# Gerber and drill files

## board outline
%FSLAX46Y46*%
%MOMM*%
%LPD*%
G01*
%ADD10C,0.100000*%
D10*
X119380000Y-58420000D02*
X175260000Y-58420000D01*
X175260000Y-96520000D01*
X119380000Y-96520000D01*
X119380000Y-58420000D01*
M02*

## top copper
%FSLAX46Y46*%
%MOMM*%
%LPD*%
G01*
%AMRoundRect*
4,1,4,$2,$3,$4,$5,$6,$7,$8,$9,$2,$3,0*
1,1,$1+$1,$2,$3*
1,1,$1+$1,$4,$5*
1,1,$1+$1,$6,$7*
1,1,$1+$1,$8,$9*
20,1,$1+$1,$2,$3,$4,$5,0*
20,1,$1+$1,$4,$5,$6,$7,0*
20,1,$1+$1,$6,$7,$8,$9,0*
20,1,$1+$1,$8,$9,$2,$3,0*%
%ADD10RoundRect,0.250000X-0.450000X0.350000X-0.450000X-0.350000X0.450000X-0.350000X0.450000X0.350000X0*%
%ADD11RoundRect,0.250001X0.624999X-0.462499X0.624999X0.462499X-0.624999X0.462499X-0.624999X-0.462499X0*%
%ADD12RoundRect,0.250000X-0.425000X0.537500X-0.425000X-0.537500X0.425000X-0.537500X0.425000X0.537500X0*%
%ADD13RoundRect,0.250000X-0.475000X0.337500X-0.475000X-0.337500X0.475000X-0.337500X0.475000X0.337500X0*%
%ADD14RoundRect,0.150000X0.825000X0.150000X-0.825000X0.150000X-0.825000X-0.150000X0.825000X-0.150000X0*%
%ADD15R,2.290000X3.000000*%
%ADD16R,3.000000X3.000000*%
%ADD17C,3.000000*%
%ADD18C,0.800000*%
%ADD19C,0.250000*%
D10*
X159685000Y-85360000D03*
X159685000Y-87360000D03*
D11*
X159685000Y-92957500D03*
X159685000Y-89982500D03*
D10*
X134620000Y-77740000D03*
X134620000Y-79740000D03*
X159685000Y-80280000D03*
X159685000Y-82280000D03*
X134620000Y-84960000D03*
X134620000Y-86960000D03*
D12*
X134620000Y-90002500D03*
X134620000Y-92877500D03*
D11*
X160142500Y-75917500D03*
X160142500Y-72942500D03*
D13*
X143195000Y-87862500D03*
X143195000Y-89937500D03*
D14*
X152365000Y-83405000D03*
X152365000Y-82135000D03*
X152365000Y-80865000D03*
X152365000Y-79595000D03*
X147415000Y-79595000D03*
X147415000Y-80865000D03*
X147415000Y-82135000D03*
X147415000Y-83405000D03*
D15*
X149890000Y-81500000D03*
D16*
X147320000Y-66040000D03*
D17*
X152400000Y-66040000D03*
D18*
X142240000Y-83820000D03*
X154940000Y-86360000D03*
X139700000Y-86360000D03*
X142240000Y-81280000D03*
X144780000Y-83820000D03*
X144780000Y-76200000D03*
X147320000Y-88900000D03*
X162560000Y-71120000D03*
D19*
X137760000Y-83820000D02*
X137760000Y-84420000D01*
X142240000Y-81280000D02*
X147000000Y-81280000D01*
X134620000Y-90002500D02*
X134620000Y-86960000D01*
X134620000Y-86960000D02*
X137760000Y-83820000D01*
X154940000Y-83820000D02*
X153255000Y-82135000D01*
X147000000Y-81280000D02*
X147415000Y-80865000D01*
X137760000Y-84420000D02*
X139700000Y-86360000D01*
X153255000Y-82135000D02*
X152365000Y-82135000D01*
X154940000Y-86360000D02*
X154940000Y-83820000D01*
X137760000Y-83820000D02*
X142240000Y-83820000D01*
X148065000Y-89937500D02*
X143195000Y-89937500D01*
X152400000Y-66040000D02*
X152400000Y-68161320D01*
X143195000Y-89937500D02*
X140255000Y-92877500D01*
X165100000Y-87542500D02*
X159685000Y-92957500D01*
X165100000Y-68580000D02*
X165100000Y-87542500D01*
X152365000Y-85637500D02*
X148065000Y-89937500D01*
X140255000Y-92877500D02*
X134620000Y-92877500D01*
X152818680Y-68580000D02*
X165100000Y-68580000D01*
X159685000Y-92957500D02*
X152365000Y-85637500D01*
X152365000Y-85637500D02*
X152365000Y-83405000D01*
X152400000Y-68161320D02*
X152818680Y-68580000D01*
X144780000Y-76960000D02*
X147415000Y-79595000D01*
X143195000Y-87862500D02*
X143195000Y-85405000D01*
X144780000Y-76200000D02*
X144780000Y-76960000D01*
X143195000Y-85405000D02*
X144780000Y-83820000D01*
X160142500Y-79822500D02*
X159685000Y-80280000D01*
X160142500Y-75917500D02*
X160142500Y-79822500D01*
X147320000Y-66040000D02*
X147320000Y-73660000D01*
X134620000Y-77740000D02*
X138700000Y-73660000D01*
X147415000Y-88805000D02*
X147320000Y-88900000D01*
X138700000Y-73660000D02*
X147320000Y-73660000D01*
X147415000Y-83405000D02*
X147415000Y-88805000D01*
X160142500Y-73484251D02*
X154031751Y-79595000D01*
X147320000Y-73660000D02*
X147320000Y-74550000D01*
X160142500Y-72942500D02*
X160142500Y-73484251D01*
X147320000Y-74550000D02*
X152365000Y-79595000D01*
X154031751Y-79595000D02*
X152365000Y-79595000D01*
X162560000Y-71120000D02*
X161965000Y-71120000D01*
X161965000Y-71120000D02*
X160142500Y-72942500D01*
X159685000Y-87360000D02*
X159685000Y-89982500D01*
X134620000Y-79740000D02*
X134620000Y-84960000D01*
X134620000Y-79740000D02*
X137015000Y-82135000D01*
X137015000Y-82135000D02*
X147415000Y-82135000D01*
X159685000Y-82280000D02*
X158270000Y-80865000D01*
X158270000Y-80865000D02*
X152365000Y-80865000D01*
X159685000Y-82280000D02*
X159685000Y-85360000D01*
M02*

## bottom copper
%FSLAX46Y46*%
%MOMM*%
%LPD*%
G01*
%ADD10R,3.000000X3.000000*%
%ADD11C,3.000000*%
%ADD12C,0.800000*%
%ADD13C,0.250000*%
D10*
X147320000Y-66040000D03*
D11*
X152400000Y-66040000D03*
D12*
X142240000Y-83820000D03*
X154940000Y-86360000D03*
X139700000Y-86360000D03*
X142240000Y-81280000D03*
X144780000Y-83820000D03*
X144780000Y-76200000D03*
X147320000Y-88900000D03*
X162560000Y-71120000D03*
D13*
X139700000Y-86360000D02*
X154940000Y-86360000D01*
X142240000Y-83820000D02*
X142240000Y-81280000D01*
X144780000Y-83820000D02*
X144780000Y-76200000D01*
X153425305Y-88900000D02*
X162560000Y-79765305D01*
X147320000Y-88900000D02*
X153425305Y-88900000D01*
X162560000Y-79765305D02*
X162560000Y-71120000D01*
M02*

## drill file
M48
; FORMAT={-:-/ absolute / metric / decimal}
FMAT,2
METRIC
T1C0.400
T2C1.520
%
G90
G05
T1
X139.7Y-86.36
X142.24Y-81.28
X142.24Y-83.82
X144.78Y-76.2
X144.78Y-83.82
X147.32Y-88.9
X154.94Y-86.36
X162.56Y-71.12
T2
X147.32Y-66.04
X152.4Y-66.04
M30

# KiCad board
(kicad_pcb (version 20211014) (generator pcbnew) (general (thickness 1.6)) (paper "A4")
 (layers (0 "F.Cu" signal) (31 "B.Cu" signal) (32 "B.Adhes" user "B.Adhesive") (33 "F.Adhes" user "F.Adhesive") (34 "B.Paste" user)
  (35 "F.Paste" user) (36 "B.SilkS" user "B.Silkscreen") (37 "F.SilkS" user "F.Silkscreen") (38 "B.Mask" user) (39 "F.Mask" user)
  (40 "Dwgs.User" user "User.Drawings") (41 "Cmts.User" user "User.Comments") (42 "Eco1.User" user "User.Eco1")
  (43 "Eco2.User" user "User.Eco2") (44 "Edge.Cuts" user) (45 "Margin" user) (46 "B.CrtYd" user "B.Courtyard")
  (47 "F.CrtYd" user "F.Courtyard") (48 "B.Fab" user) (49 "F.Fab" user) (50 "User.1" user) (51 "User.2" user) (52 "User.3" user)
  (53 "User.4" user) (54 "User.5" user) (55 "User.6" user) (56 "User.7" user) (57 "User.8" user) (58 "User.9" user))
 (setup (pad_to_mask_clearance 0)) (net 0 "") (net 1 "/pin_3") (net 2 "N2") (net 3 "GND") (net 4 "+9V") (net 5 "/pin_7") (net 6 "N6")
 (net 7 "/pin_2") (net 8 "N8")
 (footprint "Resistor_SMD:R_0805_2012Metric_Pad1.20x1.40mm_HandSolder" (layer "F.Cu") (at 159.685 86.36 -90)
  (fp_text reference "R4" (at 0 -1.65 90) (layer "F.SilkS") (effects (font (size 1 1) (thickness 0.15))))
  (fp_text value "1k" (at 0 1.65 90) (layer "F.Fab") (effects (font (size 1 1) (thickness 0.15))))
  (pad "1" smd roundrect (at -1 0 270) (size 1.2 1.4) (layers "F.Cu" "F.Paste" "F.Mask") (roundrect_rratio 0.208333) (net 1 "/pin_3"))
  (pad "2" smd roundrect (at 1 0 270) (size 1.2 1.4) (layers "F.Cu" "F.Paste" "F.Mask") (roundrect_rratio 0.208333) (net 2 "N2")))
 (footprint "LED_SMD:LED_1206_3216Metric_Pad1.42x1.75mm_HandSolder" (layer "F.Cu") (at 159.685 91.47 90)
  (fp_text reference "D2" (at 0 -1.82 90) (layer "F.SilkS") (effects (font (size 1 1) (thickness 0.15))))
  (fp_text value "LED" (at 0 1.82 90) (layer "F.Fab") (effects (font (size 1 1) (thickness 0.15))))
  (pad "1" smd roundrect (at -1.4875 0 90) (size 1.425 1.75) (layers "F.Cu" "F.Paste" "F.Mask") (roundrect_rratio 0.175439) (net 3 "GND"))
  (pad "2" smd roundrect (at 1.4875 0 90) (size 1.425 1.75) (layers "F.Cu" "F.Paste" "F.Mask") (roundrect_rratio 0.175439) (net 2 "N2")))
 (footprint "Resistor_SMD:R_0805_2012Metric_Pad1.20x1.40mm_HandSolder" (layer "F.Cu") (at 134.62 78.74 -90)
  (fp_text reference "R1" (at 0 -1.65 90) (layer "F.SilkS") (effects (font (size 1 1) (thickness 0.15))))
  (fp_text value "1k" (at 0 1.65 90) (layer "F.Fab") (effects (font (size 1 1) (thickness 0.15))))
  (pad "1" smd roundrect (at -1 0 270) (size 1.2 1.4) (layers "F.Cu" "F.Paste" "F.Mask") (roundrect_rratio 0.208333) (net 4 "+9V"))
  (pad "2" smd roundrect (at 1 0 270) (size 1.2 1.4) (layers "F.Cu" "F.Paste" "F.Mask") (roundrect_rratio 0.208333) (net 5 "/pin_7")))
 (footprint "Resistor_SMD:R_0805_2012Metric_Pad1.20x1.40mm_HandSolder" (layer "F.Cu") (at 159.685 81.28 -90)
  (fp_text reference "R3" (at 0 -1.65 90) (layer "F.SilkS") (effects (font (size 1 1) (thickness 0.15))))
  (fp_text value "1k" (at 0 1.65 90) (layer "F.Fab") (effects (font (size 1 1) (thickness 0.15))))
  (pad "1" smd roundrect (at -1 0 270) (size 1.2 1.4) (layers "F.Cu" "F.Paste" "F.Mask") (roundrect_rratio 0.208333) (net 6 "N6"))
  (pad "2" smd roundrect (at 1 0 270) (size 1.2 1.4) (layers "F.Cu" "F.Paste" "F.Mask") (roundrect_rratio 0.208333) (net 1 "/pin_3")))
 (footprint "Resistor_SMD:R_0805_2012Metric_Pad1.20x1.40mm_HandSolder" (layer "F.Cu") (at 134.62 85.96 -90)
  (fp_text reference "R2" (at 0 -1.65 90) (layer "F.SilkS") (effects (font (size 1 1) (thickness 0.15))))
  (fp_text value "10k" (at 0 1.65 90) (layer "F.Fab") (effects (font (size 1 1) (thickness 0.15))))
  (pad "1" smd roundrect (at -1 0 270) (size 1.2 1.4) (layers "F.Cu" "F.Paste" "F.Mask") (roundrect_rratio 0.208333) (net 5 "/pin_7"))
  (pad "2" smd roundrect (at 1 0 270) (size 1.2 1.4) (layers "F.Cu" "F.Paste" "F.Mask") (roundrect_rratio 0.208333) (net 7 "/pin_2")))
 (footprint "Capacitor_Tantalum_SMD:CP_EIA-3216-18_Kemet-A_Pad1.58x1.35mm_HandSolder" (layer "F.Cu") (at 134.62 91.44 -90)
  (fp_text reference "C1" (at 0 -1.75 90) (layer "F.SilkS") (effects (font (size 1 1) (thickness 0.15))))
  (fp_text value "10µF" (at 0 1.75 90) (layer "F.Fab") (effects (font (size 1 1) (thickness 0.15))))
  (pad "1" smd roundrect (at -1.4375 0 270) (size 1.575 1.35) (layers "F.Cu" "F.Paste" "F.Mask") (roundrect_rratio 0.185185)
   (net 7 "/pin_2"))
  (pad "2" smd roundrect (at 1.4375 0 270) (size 1.575 1.35) (layers "F.Cu" "F.Paste" "F.Mask") (roundrect_rratio 0.185185) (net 3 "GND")))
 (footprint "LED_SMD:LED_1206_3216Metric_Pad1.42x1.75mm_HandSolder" (layer "F.Cu") (at 160.1425 74.43 90)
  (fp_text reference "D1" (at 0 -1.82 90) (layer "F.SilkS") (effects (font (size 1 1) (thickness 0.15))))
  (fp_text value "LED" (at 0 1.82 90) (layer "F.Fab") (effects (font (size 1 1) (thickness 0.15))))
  (pad "1" smd roundrect (at -1.4875 0 90) (size 1.425 1.75) (layers "F.Cu" "F.Paste" "F.Mask") (roundrect_rratio 0.175439) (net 6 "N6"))
  (pad "2" smd roundrect (at 1.4875 0 90) (size 1.425 1.75) (layers "F.Cu" "F.Paste" "F.Mask") (roundrect_rratio 0.175439) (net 4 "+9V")))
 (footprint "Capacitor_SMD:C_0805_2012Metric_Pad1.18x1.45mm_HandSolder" (layer "F.Cu") (at 143.195 88.9 -90)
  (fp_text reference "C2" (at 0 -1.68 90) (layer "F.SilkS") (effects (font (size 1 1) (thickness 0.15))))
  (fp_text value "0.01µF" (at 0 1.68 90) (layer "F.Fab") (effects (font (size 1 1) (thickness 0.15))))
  (pad "1" smd roundrect (at -1.0375 0 270) (size 1.175 1.45) (layers "F.Cu" "F.Paste" "F.Mask") (roundrect_rratio 0.212766) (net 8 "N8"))
  (pad "2" smd roundrect (at 1.0375 0 270) (size 1.175 1.45) (layers "F.Cu" "F.Paste" "F.Mask") (roundrect_rratio 0.212766) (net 3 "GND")))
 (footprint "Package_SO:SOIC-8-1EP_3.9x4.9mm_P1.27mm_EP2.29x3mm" (layer "F.Cu") (at 149.89 81.5 180)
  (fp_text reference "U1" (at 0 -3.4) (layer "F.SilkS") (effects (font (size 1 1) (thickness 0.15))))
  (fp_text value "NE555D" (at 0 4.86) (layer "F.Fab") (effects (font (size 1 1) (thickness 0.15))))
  (pad "" smd roundrect (at 0.57 0.75 180) (size 0.92 1.21) (layers "F.Paste") (roundrect_rratio 0.25))
  (pad "" smd roundrect (at 0.57 -0.75 180) (size 0.92 1.21) (layers "F.Paste") (roundrect_rratio 0.25))
  (pad "" smd roundrect (at -0.57 0.75 180) (size 0.92 1.21) (layers "F.Paste") (roundrect_rratio 0.25))
  (pad "" smd roundrect (at -0.57 -0.75 180) (size 0.92 1.21) (layers "F.Paste") (roundrect_rratio 0.25))
  (pad "1" smd roundrect (at -2.475 -1.905 180) (size 1.95 0.6) (layers "F.Cu" "F.Paste" "F.Mask") (roundrect_rratio 0.25) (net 3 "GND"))
  (pad "2" smd roundrect (at -2.475 -0.635 180) (size 1.95 0.6) (layers "F.Cu" "F.Paste" "F.Mask") (roundrect_rratio 0.25) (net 7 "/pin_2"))
  (pad "3" smd roundrect (at -2.475 0.635 180) (size 1.95 0.6) (layers "F.Cu" "F.Paste" "F.Mask") (roundrect_rratio 0.25) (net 1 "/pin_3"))
  (pad "4" smd roundrect (at -2.475 1.905 180) (size 1.95 0.6) (layers "F.Cu" "F.Paste" "F.Mask") (roundrect_rratio 0.25) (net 4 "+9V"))
  (pad "5" smd roundrect (at 2.475 1.905 180) (size 1.95 0.6) (layers "F.Cu" "F.Paste" "F.Mask") (roundrect_rratio 0.25) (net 8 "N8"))
  (pad "6" smd roundrect (at 2.475 0.635 180) (size 1.95 0.6) (layers "F.Cu" "F.Paste" "F.Mask") (roundrect_rratio 0.25) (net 7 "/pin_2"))
  (pad "7" smd roundrect (at 2.475 -0.635 180) (size 1.95 0.6) (layers "F.Cu" "F.Paste" "F.Mask") (roundrect_rratio 0.25) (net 5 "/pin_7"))
  (pad "8" smd roundrect (at 2.475 -1.905 180) (size 1.95 0.6) (layers "F.Cu" "F.Paste" "F.Mask") (roundrect_rratio 0.25) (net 4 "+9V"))
  (pad "9" smd rect (at 0 0 180) (size 2.29 3) (layers "F.Cu" "F.Mask")))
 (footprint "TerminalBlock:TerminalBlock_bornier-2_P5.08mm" (layer "F.Cu") (at 147.32 66.04)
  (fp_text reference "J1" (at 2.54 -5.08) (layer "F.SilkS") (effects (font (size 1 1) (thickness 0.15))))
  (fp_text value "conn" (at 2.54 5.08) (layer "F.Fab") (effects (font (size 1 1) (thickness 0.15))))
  (pad "1" thru_hole rect (at 0 0) (size 3 3) (drill 1.52) (layers *.Cu *.Mask) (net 4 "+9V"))
  (pad "2" thru_hole circle (at 5.08 0) (size 3 3) (drill 1.52) (layers *.Cu *.Mask) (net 3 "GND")))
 (gr_rect (start 119.38 58.42) (end 175.26 96.52) (layer "Edge.Cuts") (width 0.1) (fill none))
 (segment (start 137.76 83.82) (end 137.76 84.42) (width 0.25) (layer "F.Cu") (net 7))
 (segment (start 142.24 81.28) (end 147 81.28) (width 0.25) (layer "F.Cu") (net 7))
 (segment (start 134.62 90.0025) (end 134.62 86.96) (width 0.25) (layer "F.Cu") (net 7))
 (segment (start 134.62 86.96) (end 137.76 83.82) (width 0.25) (layer "F.Cu") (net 7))
 (segment (start 154.94 83.82) (end 153.255 82.135) (width 0.25) (layer "F.Cu") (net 7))
 (segment (start 147 81.28) (end 147.415 80.865) (width 0.25) (layer "F.Cu") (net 7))
 (segment (start 137.76 84.42) (end 139.7 86.36) (width 0.25) (layer "F.Cu") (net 7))
 (segment (start 153.255 82.135) (end 152.365 82.135) (width 0.25) (layer "F.Cu") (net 7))
 (segment (start 154.94 86.36) (end 154.94 83.82) (width 0.25) (layer "F.Cu") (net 7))
 (segment (start 137.76 83.82) (end 142.24 83.82) (width 0.25) (layer "F.Cu") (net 7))
 (via (at 142.24 83.82) (size 0.8) (drill 0.4) (layers "F.Cu" "B.Cu") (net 7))
 (via (at 154.94 86.36) (size 0.8) (drill 0.4) (layers "F.Cu" "B.Cu") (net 7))
 (via (at 139.7 86.36) (size 0.8) (drill 0.4) (layers "F.Cu" "B.Cu") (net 7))
 (via (at 142.24 81.28) (size 0.8) (drill 0.4) (layers "F.Cu" "B.Cu") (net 7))
 (segment (start 139.7 86.36) (end 154.94 86.36) (width 0.25) (layer "B.Cu") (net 7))
 (segment (start 142.24 83.82) (end 142.24 81.28) (width 0.25) (layer "B.Cu") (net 7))
 (segment (start 148.065 89.9375) (end 143.195 89.9375) (width 0.25) (layer "F.Cu") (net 3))
 (segment (start 152.4 66.04) (end 152.4 68.16132) (width 0.25) (layer "F.Cu") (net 3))
 (segment (start 143.195 89.9375) (end 140.255 92.8775) (width 0.25) (layer "F.Cu") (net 3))
 (segment (start 165.1 87.5425) (end 159.685 92.9575) (width 0.25) (layer "F.Cu") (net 3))
 (segment (start 165.1 68.58) (end 165.1 87.5425) (width 0.25) (layer "F.Cu") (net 3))
 (segment (start 152.365 85.6375) (end 148.065 89.9375) (width 0.25) (layer "F.Cu") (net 3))
 (segment (start 140.255 92.8775) (end 134.62 92.8775) (width 0.25) (layer "F.Cu") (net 3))
 (segment (start 152.81868 68.58) (end 165.1 68.58) (width 0.25) (layer "F.Cu") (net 3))
 (segment (start 159.685 92.9575) (end 152.365 85.6375) (width 0.25) (layer "F.Cu") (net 3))
 (segment (start 152.365 85.6375) (end 152.365 83.405) (width 0.25) (layer "F.Cu") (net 3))
 (segment (start 152.4 68.16132) (end 152.81868 68.58) (width 0.25) (layer "F.Cu") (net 3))
 (segment (start 144.78 76.96) (end 147.415 79.595) (width 0.25) (layer "F.Cu") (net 8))
 (segment (start 143.195 87.8625) (end 143.195 85.405) (width 0.25) (layer "F.Cu") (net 8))
 (segment (start 144.78 76.2) (end 144.78 76.96) (width 0.25) (layer "F.Cu") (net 8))
 (segment (start 143.195 85.405) (end 144.78 83.82) (width 0.25) (layer "F.Cu") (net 8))
 (via (at 144.78 83.82) (size 0.8) (drill 0.4) (layers "F.Cu" "B.Cu") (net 8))
 (via (at 144.78 76.2) (size 0.8) (drill 0.4) (layers "F.Cu" "B.Cu") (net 8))
 (segment (start 144.78 83.82) (end 144.78 76.2) (width 0.25) (layer "B.Cu") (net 8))
 (segment (start 160.1425 79.8225) (end 159.685 80.28) (width 0.25) (layer "F.Cu") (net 6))
 (segment (start 160.1425 75.9175) (end 160.1425 79.8225) (width 0.25) (layer "F.Cu") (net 6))
 (segment (start 147.32 66.04) (end 147.32 73.66) (width 0.25) (layer "F.Cu") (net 4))
 (segment (start 134.62 77.74) (end 138.7 73.66) (width 0.25) (layer "F.Cu") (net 4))
 (segment (start 147.415 88.805) (end 147.32 88.9) (width 0.25) (layer "F.Cu") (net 4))
 (segment (start 138.7 73.66) (end 147.32 73.66) (width 0.25) (layer "F.Cu") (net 4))
 (segment (start 147.415 83.405) (end 147.415 88.805) (width 0.25) (layer "F.Cu") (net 4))
 (segment (start 160.1425 73.484251) (end 154.031751 79.595) (width 0.25) (layer "F.Cu") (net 4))
 (segment (start 147.32 73.66) (end 147.32 74.55) (width 0.25) (layer "F.Cu") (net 4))
 (segment (start 160.1425 72.9425) (end 160.1425 73.484251) (width 0.25) (layer "F.Cu") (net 4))
 (segment (start 147.32 74.55) (end 152.365 79.595) (width 0.25) (layer "F.Cu") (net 4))
 (segment (start 154.031751 79.595) (end 152.365 79.595) (width 0.25) (layer "F.Cu") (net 4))
 (segment (start 162.56 71.12) (end 161.965 71.12) (width 0.25) (layer "F.Cu") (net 4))
 (segment (start 161.965 71.12) (end 160.1425 72.9425) (width 0.25) (layer "F.Cu") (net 4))
 (via (at 147.32 88.9) (size 0.8) (drill 0.4) (layers "F.Cu" "B.Cu") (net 4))
 (via (at 162.56 71.12) (size 0.8) (drill 0.4) (layers "F.Cu" "B.Cu") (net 4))
 (segment (start 153.425305 88.9) (end 162.56 79.765305) (width 0.25) (layer "B.Cu") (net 4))
 (segment (start 147.32 88.9) (end 153.425305 88.9) (width 0.25) (layer "B.Cu") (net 4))
 (segment (start 162.56 79.765305) (end 162.56 71.12) (width 0.25) (layer "B.Cu") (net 4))
 (segment (start 159.685 87.36) (end 159.685 89.9825) (width 0.25) (layer "F.Cu") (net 2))
 (segment (start 134.62 79.74) (end 134.62 84.96) (width 0.25) (layer "F.Cu") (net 5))
 (segment (start 134.62 79.74) (end 137.015 82.135) (width 0.25) (layer "F.Cu") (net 5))
 (segment (start 137.015 82.135) (end 147.415 82.135) (width 0.25) (layer "F.Cu") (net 5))
 (segment (start 159.685 82.28) (end 158.27 80.865) (width 0.25) (layer "F.Cu") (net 1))
 (segment (start 158.27 80.865) (end 152.365 80.865) (width 0.25) (layer "F.Cu") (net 1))
 (segment (start 159.685 82.28) (end 159.685 85.36) (width 0.25) (layer "F.Cu") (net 1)))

